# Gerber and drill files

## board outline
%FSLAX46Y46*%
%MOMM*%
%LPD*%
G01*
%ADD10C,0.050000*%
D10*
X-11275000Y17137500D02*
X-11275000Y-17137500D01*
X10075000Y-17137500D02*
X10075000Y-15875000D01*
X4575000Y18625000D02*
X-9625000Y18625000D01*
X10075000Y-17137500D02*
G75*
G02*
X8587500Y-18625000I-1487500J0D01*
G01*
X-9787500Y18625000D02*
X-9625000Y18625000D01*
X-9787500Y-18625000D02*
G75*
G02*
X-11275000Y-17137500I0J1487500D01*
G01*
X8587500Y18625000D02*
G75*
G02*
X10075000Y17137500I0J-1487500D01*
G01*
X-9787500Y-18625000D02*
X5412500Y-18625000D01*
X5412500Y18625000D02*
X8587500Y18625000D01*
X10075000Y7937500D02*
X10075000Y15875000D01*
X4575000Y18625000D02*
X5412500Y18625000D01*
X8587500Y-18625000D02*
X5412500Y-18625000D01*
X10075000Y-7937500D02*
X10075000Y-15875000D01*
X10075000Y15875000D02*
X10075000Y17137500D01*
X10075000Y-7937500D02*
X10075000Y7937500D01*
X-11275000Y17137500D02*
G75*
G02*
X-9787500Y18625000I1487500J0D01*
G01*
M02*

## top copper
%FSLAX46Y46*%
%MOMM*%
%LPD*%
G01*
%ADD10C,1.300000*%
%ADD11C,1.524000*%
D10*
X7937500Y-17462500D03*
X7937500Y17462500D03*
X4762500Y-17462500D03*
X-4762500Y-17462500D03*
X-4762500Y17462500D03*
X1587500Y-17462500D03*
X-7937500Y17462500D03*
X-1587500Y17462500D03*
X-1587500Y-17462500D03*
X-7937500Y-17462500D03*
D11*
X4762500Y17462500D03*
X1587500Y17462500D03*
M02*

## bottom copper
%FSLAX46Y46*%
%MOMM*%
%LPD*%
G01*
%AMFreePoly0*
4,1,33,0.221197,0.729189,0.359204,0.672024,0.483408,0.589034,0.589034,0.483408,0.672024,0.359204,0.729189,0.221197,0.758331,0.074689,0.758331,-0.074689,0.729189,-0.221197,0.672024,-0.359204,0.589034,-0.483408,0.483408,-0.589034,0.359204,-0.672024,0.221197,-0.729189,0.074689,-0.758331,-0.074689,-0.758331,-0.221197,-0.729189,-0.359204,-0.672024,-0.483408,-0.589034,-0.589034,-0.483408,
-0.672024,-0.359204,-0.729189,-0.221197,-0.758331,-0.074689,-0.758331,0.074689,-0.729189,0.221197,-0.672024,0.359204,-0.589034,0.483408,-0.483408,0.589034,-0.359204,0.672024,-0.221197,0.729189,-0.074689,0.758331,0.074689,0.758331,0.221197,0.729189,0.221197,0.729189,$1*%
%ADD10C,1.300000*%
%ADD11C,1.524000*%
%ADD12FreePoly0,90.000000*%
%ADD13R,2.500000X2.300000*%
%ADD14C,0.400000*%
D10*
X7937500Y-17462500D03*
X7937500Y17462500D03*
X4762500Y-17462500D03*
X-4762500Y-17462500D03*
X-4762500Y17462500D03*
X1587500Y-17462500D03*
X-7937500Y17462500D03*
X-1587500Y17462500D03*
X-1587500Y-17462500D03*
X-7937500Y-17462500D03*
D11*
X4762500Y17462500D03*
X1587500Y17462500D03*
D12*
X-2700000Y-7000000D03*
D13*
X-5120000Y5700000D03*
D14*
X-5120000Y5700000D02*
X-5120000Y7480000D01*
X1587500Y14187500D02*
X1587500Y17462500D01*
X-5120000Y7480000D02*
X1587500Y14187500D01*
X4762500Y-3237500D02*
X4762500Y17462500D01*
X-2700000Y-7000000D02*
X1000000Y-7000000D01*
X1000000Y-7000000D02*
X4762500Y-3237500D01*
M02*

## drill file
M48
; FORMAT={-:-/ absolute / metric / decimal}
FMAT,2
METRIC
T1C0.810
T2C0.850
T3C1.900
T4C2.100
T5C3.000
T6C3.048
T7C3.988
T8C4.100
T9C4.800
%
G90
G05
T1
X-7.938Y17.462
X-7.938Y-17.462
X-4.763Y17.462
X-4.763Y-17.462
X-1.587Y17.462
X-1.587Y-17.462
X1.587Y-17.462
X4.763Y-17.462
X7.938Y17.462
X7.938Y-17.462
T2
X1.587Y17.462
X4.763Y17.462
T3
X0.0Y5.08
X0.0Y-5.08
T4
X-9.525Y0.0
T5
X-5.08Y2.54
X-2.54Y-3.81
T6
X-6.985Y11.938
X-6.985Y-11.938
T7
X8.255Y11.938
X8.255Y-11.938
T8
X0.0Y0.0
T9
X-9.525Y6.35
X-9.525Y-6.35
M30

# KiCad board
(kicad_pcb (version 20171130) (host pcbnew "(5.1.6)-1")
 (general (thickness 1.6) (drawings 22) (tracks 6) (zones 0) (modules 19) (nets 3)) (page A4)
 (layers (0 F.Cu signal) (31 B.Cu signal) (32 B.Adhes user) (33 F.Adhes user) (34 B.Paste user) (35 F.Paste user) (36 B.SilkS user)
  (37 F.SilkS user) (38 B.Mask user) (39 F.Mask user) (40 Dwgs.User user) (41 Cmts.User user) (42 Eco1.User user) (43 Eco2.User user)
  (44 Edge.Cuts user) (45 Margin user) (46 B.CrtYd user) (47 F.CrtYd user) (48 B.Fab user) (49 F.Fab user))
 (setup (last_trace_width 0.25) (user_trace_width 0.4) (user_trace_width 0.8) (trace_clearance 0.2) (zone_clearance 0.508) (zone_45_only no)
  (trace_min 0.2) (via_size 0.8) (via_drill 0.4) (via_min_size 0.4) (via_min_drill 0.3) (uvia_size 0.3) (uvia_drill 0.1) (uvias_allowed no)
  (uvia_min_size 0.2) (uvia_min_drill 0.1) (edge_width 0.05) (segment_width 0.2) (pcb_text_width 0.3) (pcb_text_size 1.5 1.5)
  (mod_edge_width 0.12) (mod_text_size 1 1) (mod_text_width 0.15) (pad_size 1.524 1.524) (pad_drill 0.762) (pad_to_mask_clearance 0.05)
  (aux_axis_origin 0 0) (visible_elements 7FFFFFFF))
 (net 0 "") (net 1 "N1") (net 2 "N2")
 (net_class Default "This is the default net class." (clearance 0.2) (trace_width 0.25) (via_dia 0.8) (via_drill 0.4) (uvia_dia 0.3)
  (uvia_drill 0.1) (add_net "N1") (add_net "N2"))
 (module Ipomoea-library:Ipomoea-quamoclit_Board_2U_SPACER (layer F.Cu) (at 0 0 90)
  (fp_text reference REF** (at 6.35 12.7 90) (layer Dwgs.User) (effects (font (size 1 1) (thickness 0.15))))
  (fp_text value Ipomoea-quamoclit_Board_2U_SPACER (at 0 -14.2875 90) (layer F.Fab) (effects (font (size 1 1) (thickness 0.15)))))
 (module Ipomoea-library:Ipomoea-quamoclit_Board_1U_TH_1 (layer F.Cu) (at 7.9375 17.4625)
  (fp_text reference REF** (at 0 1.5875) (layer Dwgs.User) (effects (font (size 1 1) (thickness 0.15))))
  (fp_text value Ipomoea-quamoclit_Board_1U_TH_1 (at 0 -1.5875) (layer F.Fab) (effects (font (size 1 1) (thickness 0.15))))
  (pad "" thru_hole circle (at 0 0 180) (size 1.3 1.3) (drill 0.81) (layers *.Cu *.Mask)))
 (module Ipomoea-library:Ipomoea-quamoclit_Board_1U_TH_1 (layer F.Cu) (at 7.9375 -17.4625)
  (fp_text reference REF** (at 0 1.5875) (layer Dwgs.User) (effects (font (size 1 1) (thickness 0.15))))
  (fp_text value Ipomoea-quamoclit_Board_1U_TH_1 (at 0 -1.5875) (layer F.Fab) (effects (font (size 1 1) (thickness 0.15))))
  (pad "" thru_hole circle (at 0 0 180) (size 1.3 1.3) (drill 0.81) (layers *.Cu *.Mask)))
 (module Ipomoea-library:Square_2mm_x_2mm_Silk (layer F.Cu) (at 4.7625 -17.4625)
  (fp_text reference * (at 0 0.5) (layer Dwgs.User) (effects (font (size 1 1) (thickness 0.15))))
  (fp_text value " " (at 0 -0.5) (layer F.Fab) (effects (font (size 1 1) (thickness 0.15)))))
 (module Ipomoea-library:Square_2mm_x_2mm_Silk (layer F.Cu) (at 1.5875 -17.4625)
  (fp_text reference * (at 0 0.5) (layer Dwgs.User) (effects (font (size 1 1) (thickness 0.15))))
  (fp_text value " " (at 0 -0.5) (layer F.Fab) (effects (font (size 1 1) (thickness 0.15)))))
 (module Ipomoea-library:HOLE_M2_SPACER (layer F.Cu) (at -9.525 6.35)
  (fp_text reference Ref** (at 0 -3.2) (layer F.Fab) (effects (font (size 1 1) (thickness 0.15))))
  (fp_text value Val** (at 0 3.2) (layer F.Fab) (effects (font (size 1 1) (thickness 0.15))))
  (pad "" np_thru_hole circle (at 0 0) (size 4.8 4.8) (drill 4.8) (layers *.Cu *.Mask)))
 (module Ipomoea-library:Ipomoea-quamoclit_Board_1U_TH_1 (layer F.Cu) (at 4.7625 17.4625)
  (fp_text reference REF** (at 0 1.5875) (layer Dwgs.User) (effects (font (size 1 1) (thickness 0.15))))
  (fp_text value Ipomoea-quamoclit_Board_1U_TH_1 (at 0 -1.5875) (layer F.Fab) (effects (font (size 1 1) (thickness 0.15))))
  (pad "" thru_hole circle (at 0 0 180) (size 1.3 1.3) (drill 0.81) (layers *.Cu *.Mask)))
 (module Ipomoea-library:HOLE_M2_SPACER (layer F.Cu) (at -9.525 -6.35)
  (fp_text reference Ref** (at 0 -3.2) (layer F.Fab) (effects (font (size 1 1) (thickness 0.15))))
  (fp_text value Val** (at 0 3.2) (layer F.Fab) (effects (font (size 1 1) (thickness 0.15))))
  (pad "" np_thru_hole circle (at 0 0) (size 4.8 4.8) (drill 4.8) (layers *.Cu *.Mask)))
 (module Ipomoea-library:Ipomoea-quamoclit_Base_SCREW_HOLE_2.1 (layer F.Cu) (at -9.525 0)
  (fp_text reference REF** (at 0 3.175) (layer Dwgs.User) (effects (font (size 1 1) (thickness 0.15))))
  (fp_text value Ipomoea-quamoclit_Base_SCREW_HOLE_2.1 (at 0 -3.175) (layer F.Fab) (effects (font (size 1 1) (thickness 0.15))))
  (pad "" np_thru_hole circle (at 0 0) (size 2.1 2.1) (drill 2.1) (layers *.Cu *.Mask)))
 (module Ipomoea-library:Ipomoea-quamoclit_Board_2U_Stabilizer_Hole (layer F.Cu) (at 0 0 90)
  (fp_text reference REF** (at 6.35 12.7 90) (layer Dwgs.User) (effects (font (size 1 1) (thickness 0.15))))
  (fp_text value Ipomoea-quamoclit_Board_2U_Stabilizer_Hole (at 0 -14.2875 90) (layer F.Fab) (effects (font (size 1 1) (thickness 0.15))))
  (pad "" np_thru_hole circle (at 11.938 8.255 90) (size 3.9878 3.9878) (drill 3.9878) (layers *.Cu *.Mask))
  (pad "" np_thru_hole circle (at -11.938 8.255 90) (size 3.9878 3.9878) (drill 3.9878) (layers *.Cu *.Mask))
  (pad "" np_thru_hole circle (at 11.938 -6.985 90) (size 3.048 3.048) (drill 3.048) (layers *.Cu *.Mask))
  (pad "" np_thru_hole circle (at -11.938 -6.985 90) (size 3.048 3.048) (drill 3.048) (layers *.Cu *.Mask)))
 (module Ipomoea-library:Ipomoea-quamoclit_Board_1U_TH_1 (layer F.Cu) (at -4.7625 17.4625)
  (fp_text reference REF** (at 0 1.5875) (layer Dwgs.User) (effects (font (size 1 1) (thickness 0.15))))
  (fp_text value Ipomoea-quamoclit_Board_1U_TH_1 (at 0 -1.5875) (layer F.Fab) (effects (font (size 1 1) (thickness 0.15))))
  (pad "" thru_hole circle (at 0 0 180) (size 1.3 1.3) (drill 0.81) (layers *.Cu *.Mask)))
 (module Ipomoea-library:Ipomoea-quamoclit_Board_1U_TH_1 (layer F.Cu) (at -4.7625 -17.4625)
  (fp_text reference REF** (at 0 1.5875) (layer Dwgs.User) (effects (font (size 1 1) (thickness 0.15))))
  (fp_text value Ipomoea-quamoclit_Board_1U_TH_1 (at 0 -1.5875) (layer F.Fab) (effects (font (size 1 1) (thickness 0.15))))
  (pad "" thru_hole circle (at 0 0 180) (size 1.3 1.3) (drill 0.81) (layers *.Cu *.Mask)))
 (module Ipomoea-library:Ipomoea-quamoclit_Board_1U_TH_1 (layer F.Cu) (at 1.5875 17.4625)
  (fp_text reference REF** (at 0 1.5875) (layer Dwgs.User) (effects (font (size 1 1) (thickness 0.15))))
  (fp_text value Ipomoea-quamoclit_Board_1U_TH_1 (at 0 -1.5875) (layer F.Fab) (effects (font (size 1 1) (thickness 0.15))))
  (pad "" thru_hole circle (at 0 0 180) (size 1.3 1.3) (drill 0.81) (layers *.Cu *.Mask)))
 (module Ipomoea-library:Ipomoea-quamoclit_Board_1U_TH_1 (layer F.Cu) (at -7.9375 -17.4625)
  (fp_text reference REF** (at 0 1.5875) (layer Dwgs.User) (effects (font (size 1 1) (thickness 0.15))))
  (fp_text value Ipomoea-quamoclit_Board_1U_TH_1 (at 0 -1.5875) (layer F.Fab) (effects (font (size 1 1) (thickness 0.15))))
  (pad "" thru_hole circle (at 0 0 180) (size 1.3 1.3) (drill 0.81) (layers *.Cu *.Mask)))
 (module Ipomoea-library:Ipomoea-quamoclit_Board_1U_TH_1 (layer F.Cu) (at -1.5875 -17.4625)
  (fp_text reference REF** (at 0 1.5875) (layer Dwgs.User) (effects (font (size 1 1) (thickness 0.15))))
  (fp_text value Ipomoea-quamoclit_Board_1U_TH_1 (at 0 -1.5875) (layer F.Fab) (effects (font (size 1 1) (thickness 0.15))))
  (pad "" thru_hole circle (at 0 0 180) (size 1.3 1.3) (drill 0.81) (layers *.Cu *.Mask)))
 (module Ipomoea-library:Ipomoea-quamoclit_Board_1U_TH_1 (layer F.Cu) (at -1.5875 17.4625)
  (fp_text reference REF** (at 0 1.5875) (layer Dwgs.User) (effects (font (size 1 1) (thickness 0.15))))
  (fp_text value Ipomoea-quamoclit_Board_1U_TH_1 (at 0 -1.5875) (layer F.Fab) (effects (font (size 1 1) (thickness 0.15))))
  (pad "" thru_hole circle (at 0 0 180) (size 1.3 1.3) (drill 0.81) (layers *.Cu *.Mask)))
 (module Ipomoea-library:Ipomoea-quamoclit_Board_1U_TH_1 (layer F.Cu) (at -7.9375 17.4625)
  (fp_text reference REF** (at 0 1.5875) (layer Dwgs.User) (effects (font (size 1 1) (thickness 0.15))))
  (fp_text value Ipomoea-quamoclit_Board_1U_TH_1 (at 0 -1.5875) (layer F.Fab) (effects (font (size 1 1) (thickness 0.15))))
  (pad "" thru_hole circle (at 0 0 180) (size 1.3 1.3) (drill 0.81) (layers *.Cu *.Mask)))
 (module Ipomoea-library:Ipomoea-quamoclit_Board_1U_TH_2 (layer F.Cu) (at 3.175 -17.4625 180)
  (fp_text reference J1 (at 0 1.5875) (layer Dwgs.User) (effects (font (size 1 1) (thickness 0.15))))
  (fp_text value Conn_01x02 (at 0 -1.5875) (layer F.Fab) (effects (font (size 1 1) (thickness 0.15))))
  (pad 1 thru_hole circle (at -1.5875 0) (size 1.524 1.524) (drill 0.85) (layers *.Cu *.Mask) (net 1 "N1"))
  (pad 2 thru_hole circle (at 1.5875 0) (size 1.524 1.524) (drill 0.85) (layers *.Cu *.Mask) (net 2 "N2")))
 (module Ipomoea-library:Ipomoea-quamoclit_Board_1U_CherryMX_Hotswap (layer F.Cu) (at 0 0 90)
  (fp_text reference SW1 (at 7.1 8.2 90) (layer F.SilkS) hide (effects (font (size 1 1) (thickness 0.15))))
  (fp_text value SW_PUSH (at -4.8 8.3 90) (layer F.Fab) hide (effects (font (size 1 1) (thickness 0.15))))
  (pad "" np_thru_hole circle (at 0 0 180) (size 4.1 4.1) (drill 4.1) (layers *.Cu *.Mask))
  (pad "" np_thru_hole circle (at 5.08 0 90) (size 1.9 1.9) (drill 1.9) (layers *.Cu *.Mask))
  (pad "" np_thru_hole circle (at -5.08 0 90) (size 1.9 1.9) (drill 1.9) (layers *.Cu *.Mask))
  (pad 1 smd custom (at -7 -2.7 90) (size 1.524 1.524) (layers B.Cu B.Paste B.Mask) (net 1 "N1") (zone_connect 0)
   (options (clearance outline) (anchor circle)) (primitives))
  (pad "" np_thru_hole circle (at 2.54 -5.08 270) (size 3 3) (drill 3) (layers *.Cu *.Mask))
  (pad 2 smd rect (at 5.7 -5.12 270) (size 2.3 2.5) (layers B.Cu B.Paste B.Mask) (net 2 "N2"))
  (pad "" np_thru_hole circle (at -3.81 -2.54 270) (size 3 3) (drill 3) (layers *.Cu *.Mask)))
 (gr_line (start -11.275 -17.1375) (end -11.275 17.1375) (layer Edge.Cuts) (width 0.05))
 (gr_line (start 10.075 17.1375) (end 10.075 15.875) (layer Edge.Cuts) (width 0.05))
 (gr_line (start 4.575 -18.625) (end -9.625 -18.625) (layer Edge.Cuts) (width 0.05))
 (gr_arc (start 8.5875 17.1375) (end 8.5875 18.625) (angle -90) (layer Edge.Cuts) (width 0.05))
 (gr_line (start -9.7875 -18.625) (end -9.625 -18.625) (layer Edge.Cuts) (width 0.05))
 (gr_arc (start -9.7875 17.1375) (end -11.275 17.1375) (angle -90) (layer Edge.Cuts) (width 0.05))
 (gr_arc (start 8.5875 -17.1375) (end 10.075 -17.1375) (angle -90) (layer Edge.Cuts) (width 0.05))
 (gr_line (start -9.7875 18.625) (end 5.4125 18.625) (layer Edge.Cuts) (width 0.05))
 (gr_line (start 5.4125 -18.625) (end 8.5875 -18.625) (layer Edge.Cuts) (width 0.05))
 (gr_line (start 10.075 -7.9375) (end 10.075 -15.875) (layer Edge.Cuts) (width 0.05))
 (gr_line (start 4.575 -18.625) (end 5.4125 -18.625) (layer Edge.Cuts) (width 0.05))
 (gr_line (start 8.5875 18.625) (end 5.4125 18.625) (layer Edge.Cuts) (width 0.05))
 (gr_line (start 10.075 7.9375) (end 10.075 15.875) (layer Edge.Cuts) (width 0.05))
 (gr_line (start 10.075 -15.875) (end 10.075 -17.1375) (layer Edge.Cuts) (width 0.05))
 (gr_line (start 10.075 7.9375) (end 10.075 -7.9375) (layer Edge.Cuts) (width 0.05))
 (gr_arc (start -9.7875 -17.1375) (end -9.7875 -18.625) (angle -90) (layer Edge.Cuts) (width 0.05))
 (segment (start -5.12 -5.7) (end -5.12 -7.48) (width 0.4) (layer B.Cu) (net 2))
 (segment (start 1.5875 -14.1875) (end 1.5875 -17.4625) (width 0.4) (layer B.Cu) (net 2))
 (segment (start -5.12 -7.48) (end 1.5875 -14.1875) (width 0.4) (layer B.Cu) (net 2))
 (segment (start 4.7625 3.2375) (end 4.7625 -17.4625) (width 0.4) (layer B.Cu) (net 1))
 (segment (start -2.7 7) (end 1 7) (width 0.4) (layer B.Cu) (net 1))
 (segment (start 1 7) (end 4.7625 3.2375) (width 0.4) (layer B.Cu) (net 1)))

